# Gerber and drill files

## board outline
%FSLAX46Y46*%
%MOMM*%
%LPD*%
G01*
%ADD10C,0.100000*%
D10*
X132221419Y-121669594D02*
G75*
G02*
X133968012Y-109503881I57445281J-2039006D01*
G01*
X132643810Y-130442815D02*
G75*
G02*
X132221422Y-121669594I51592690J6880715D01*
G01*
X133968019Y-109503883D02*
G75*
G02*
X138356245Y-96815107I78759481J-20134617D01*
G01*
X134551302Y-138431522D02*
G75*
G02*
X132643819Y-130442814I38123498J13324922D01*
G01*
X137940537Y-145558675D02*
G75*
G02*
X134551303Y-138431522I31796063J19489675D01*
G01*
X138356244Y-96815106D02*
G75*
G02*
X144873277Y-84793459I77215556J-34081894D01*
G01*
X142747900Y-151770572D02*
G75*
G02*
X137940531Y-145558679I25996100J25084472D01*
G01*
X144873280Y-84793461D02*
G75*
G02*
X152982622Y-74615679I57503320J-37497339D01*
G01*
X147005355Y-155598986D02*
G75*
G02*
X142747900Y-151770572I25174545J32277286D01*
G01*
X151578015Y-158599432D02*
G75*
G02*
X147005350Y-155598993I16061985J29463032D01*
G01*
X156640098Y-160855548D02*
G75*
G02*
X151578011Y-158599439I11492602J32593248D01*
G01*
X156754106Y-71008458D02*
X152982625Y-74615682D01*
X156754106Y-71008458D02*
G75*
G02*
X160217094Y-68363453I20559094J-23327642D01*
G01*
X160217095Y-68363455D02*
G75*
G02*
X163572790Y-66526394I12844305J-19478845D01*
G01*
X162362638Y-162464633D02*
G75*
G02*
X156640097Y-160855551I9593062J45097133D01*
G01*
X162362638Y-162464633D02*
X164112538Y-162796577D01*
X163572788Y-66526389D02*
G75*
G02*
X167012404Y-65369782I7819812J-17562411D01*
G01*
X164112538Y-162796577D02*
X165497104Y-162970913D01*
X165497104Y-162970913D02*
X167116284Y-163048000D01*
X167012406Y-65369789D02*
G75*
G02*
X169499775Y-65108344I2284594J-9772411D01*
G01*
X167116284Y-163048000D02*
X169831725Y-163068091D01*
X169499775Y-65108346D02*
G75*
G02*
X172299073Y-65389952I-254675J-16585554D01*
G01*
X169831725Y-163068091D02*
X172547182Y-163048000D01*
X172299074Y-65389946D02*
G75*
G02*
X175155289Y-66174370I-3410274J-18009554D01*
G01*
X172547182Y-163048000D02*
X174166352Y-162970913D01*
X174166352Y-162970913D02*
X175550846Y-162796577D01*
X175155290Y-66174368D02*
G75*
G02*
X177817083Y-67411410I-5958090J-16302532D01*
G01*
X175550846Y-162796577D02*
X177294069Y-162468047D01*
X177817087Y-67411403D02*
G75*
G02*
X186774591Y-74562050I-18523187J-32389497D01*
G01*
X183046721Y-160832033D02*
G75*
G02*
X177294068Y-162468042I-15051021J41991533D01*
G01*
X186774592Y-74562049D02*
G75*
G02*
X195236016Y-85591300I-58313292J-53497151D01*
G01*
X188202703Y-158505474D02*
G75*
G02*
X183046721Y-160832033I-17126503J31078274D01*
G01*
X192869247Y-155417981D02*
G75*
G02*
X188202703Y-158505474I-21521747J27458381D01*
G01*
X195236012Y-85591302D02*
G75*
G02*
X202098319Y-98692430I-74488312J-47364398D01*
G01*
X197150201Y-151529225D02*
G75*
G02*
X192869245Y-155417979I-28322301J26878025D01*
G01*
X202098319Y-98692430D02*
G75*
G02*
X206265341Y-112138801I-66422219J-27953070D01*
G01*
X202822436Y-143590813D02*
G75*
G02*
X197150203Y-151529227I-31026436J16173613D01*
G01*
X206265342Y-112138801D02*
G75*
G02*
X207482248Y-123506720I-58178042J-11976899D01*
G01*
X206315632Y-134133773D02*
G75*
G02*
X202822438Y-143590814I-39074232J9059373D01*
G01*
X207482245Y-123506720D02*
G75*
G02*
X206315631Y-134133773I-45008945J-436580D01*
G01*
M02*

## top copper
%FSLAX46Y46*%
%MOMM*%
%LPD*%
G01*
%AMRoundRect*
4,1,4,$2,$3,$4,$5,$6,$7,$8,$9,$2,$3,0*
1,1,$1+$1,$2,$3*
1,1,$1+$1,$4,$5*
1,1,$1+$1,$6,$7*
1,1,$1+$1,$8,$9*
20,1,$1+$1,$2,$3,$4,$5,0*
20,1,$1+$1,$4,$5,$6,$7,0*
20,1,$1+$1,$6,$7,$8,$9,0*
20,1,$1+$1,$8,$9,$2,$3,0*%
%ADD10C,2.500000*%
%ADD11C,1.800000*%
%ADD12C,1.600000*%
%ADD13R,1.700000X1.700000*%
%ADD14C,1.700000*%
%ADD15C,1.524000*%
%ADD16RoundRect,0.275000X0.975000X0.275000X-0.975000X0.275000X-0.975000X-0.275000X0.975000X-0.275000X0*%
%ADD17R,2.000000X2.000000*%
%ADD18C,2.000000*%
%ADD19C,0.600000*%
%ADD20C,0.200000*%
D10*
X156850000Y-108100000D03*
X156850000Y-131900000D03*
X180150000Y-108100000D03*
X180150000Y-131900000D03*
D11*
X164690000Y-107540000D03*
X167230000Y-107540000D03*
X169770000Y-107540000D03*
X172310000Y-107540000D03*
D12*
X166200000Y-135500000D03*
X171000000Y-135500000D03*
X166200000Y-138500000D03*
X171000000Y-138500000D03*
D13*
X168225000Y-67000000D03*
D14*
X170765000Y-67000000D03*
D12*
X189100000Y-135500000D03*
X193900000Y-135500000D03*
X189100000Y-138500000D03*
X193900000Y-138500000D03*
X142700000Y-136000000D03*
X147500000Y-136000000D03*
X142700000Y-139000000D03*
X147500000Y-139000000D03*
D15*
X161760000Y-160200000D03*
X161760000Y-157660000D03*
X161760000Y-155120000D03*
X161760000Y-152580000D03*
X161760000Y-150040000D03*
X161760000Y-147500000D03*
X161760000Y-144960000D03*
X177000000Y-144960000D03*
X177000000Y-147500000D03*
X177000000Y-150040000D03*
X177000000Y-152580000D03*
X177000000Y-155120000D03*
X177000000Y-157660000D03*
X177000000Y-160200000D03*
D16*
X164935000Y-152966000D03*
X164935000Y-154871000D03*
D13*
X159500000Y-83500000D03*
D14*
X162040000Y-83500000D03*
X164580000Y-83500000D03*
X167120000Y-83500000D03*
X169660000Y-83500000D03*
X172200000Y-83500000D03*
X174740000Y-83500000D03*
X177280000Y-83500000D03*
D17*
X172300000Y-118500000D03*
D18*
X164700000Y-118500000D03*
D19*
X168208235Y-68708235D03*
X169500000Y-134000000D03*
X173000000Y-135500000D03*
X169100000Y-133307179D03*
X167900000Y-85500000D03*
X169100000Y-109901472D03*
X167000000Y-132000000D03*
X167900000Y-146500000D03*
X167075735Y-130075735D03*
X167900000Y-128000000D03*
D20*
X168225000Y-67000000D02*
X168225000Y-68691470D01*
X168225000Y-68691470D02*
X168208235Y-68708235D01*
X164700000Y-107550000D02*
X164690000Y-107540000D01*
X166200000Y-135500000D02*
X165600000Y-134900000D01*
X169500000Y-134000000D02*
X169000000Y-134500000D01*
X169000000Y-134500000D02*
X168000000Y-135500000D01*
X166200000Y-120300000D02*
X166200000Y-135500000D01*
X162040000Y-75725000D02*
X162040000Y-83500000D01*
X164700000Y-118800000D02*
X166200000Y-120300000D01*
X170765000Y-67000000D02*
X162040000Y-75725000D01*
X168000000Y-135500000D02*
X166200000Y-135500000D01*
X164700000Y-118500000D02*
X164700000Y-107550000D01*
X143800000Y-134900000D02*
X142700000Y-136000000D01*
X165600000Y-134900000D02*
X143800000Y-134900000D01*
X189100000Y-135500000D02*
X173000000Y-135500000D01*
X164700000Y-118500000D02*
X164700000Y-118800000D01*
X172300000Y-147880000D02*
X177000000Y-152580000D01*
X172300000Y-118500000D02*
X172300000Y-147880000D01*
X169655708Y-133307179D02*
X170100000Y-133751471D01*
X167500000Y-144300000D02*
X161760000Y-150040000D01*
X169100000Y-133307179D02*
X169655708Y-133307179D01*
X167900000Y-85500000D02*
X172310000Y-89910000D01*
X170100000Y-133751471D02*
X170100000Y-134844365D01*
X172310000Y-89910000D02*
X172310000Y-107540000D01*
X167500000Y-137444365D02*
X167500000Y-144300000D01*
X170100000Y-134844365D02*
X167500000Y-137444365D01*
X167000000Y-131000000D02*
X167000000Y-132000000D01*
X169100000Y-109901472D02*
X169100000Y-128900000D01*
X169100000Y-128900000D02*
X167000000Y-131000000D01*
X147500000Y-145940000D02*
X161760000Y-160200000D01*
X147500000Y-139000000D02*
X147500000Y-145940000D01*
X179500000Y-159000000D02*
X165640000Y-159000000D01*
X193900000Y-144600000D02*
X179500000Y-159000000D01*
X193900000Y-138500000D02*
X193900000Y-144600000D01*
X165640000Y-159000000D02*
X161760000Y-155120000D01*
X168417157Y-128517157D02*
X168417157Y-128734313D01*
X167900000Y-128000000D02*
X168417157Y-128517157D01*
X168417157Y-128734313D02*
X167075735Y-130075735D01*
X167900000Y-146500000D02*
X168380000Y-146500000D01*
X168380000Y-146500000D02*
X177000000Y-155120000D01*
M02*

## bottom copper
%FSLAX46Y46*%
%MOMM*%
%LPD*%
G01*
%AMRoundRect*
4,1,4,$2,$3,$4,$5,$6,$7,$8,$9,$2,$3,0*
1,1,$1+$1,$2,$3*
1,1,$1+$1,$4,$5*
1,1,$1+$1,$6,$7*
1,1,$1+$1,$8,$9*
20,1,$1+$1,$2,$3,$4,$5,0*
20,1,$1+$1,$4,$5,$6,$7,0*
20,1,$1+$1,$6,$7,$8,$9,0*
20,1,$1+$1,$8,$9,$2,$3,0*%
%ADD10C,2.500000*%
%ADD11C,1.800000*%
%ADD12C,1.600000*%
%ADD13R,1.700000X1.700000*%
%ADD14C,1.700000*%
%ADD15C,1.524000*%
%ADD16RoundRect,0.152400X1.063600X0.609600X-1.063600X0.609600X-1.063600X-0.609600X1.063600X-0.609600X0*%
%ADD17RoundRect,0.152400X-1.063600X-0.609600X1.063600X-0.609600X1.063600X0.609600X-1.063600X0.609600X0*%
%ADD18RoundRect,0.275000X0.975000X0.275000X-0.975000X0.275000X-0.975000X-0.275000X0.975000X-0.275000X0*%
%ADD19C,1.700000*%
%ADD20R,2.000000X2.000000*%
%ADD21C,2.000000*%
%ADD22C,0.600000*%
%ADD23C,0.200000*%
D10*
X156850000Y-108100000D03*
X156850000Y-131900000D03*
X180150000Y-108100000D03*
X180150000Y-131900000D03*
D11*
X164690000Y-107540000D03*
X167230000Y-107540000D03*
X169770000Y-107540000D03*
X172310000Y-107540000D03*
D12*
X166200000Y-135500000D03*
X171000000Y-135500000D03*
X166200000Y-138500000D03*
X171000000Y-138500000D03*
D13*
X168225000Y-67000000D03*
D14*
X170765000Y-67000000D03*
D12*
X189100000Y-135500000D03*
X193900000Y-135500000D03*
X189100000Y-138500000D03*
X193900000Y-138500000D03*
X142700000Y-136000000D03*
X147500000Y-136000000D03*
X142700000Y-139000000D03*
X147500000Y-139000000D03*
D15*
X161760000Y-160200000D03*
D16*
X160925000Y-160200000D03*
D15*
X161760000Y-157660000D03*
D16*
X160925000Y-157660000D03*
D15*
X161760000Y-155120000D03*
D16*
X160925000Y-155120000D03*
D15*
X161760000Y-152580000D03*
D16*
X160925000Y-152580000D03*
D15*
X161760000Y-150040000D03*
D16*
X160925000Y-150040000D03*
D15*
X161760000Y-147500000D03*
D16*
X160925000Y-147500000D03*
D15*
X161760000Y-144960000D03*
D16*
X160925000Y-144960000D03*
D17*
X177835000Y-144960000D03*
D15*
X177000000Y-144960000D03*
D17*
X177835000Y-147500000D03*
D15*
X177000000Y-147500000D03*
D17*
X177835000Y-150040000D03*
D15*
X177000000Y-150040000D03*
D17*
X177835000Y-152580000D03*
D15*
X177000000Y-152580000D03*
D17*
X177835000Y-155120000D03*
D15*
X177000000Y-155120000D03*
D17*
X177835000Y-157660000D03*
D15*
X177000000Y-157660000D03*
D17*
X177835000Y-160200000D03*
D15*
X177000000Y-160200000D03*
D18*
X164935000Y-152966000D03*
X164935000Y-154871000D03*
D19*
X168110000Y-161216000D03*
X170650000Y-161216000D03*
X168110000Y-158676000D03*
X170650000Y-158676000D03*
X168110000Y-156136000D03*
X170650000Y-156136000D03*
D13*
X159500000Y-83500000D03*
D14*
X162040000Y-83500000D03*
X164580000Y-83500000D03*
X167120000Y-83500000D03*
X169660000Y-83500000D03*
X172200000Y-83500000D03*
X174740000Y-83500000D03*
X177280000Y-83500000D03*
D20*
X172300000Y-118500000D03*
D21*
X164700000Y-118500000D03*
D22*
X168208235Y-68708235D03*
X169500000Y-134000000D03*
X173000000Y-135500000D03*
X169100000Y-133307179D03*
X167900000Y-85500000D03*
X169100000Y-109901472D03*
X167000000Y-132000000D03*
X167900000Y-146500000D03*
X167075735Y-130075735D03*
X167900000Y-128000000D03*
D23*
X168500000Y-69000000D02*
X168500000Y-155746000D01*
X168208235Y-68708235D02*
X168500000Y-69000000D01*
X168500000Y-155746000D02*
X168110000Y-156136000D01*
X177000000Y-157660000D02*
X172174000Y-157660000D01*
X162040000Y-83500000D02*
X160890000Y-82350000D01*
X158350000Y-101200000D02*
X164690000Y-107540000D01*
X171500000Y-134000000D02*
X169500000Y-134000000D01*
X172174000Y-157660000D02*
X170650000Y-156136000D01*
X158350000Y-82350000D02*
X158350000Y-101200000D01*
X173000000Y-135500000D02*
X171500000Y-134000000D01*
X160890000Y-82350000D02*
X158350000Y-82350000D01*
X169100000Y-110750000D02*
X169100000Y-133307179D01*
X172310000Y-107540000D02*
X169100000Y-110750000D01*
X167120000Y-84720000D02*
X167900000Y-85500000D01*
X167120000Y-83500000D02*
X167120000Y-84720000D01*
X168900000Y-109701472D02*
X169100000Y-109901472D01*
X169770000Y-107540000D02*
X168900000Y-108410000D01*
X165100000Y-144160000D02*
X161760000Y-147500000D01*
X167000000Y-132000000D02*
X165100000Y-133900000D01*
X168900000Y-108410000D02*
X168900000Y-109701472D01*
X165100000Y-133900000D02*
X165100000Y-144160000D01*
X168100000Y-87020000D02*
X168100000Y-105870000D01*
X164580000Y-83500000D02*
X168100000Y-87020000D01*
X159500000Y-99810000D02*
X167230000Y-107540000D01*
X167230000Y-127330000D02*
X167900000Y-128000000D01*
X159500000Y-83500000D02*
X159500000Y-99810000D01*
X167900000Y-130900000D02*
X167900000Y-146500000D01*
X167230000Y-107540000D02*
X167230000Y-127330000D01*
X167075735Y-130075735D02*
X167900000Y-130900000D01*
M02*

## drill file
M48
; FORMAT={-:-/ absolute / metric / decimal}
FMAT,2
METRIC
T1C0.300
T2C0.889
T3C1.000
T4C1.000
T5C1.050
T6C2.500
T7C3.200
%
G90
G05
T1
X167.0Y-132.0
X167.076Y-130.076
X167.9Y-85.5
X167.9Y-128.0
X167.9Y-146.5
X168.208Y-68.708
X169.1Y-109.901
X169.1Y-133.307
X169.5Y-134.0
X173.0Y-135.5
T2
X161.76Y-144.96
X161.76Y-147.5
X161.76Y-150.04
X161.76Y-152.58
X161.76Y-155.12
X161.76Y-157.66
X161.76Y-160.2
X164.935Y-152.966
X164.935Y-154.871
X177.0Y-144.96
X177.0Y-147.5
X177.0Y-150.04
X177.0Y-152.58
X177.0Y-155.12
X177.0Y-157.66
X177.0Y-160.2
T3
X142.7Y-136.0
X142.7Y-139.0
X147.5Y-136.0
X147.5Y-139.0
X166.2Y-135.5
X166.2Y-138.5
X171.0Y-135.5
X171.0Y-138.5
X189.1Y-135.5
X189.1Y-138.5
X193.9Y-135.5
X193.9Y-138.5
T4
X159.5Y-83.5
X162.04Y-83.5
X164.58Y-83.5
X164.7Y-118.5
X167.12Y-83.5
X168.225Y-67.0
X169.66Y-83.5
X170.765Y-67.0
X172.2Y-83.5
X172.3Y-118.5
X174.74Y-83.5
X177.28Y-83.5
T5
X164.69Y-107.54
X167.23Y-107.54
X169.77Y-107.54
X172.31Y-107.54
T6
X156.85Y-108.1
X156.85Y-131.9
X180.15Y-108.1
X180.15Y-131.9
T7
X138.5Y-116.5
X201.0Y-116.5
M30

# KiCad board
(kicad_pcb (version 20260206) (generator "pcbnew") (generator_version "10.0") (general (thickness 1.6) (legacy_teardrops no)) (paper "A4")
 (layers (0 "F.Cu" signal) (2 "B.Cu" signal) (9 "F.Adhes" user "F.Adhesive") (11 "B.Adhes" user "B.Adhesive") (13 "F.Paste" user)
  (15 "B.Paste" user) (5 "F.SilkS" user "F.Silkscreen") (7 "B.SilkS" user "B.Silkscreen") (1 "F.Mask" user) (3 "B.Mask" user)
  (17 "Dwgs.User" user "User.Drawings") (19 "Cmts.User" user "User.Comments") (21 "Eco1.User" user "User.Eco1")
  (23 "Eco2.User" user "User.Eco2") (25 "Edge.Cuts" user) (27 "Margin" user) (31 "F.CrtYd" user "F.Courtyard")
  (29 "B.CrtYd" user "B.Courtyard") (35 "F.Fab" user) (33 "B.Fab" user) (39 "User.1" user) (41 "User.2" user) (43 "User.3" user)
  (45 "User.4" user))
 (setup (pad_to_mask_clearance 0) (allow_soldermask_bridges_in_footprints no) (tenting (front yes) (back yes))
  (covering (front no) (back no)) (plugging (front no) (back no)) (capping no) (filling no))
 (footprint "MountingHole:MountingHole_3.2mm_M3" (layer "F.Cu") (at 138.5 116.5)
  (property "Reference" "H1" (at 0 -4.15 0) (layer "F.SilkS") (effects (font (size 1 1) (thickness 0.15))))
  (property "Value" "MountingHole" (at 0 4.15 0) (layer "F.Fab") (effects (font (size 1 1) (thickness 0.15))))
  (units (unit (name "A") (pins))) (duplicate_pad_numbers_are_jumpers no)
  (pad "" np_thru_hole circle (at 0 0) (size 3.2 3.2) (drill 3.2) (layers "*.Cu" "*.Mask")))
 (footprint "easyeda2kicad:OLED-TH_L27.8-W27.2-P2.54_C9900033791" (layer "F.Cu") (at 168.5 107.54)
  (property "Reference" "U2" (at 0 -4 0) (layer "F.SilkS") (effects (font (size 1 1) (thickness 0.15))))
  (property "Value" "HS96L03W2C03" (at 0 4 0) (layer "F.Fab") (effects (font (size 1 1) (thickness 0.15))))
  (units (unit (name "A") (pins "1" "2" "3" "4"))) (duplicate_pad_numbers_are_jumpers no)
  (pad "" thru_hole circle (at -11.65 0.56) (size 2.5 2.5) (drill 2.5) (layers "*.Cu" "*.Mask") (remove_unused_layers no))
  (pad "" thru_hole circle (at -11.65 24.36) (size 2.5 2.5) (drill 2.5) (layers "*.Cu" "*.Mask") (remove_unused_layers no))
  (pad "" thru_hole circle (at 11.65 0.56) (size 2.5 2.5) (drill 2.5) (layers "*.Cu" "*.Mask") (remove_unused_layers no))
  (pad "" thru_hole circle (at 11.65 24.36) (size 2.5 2.5) (drill 2.5) (layers "*.Cu" "*.Mask") (remove_unused_layers no))
  (pad "1" thru_hole circle (at -3.81 0) (size 1.8 1.8) (drill 1.049986) (layers "*.Cu" "*.Mask") (remove_unused_layers no) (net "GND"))
  (pad "2" thru_hole circle (at -1.27 0) (size 1.8 1.8) (drill 1.049986) (layers "*.Cu" "*.Mask") (remove_unused_layers no) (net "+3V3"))
  (pad "3" thru_hole circle (at 1.27 0) (size 1.8 1.8) (drill 1.049986) (layers "*.Cu" "*.Mask") (remove_unused_layers no) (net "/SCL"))
  (pad "4" thru_hole circle (at 3.81 0) (size 1.8 1.8) (drill 1.049986) (layers "*.Cu" "*.Mask") (remove_unused_layers no) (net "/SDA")))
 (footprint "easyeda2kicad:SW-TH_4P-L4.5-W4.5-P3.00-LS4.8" (layer "F.Cu") (at 168.6 137)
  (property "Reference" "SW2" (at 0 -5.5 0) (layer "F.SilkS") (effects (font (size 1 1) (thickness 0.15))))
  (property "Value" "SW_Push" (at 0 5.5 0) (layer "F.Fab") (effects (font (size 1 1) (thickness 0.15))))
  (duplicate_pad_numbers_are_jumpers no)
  (pad "1" thru_hole circle (at -2.4 -1.5) (size 1.6 1.6) (drill 0.999998) (layers "*.Cu" "*.Mask") (remove_unused_layers no) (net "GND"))
  (pad "1" thru_hole circle (at 2.4 -1.5) (size 1.6 1.6) (drill 0.999998) (layers "*.Cu" "*.Mask") (remove_unused_layers no))
  (pad "2" thru_hole circle (at -2.4 1.5) (size 1.6 1.6) (drill 0.999998) (layers "*.Cu" "*.Mask") (remove_unused_layers no))
  (pad "2" thru_hole circle (at 2.4 1.5) (size 1.6 1.6) (drill 0.999998) (layers "*.Cu" "*.Mask") (remove_unused_layers no)
   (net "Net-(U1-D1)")))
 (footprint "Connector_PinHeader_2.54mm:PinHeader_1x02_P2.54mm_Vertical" (layer "F.Cu") (at 168.225 67 90)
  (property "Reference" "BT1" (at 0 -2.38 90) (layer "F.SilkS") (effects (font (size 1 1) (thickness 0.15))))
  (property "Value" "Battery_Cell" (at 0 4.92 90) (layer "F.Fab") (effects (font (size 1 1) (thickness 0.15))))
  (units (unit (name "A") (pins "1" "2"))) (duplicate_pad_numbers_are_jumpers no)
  (pad "1" thru_hole rect (at 0 0 90) (size 1.7 1.7) (drill 1) (layers "*.Cu" "*.Mask") (remove_unused_layers no) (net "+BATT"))
  (pad "2" thru_hole circle (at 0 2.54 90) (size 1.7 1.7) (drill 1) (layers "*.Cu" "*.Mask") (remove_unused_layers no) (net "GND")))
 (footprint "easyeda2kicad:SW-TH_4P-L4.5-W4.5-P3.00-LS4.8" (layer "F.Cu") (at 191.5 137)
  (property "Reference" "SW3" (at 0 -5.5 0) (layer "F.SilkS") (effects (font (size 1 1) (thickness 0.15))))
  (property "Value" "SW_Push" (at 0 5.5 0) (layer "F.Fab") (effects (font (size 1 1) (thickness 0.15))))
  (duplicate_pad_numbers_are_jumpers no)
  (pad "1" thru_hole circle (at -2.4 -1.5) (size 1.6 1.6) (drill 0.999998) (layers "*.Cu" "*.Mask") (remove_unused_layers no) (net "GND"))
  (pad "1" thru_hole circle (at 2.4 -1.5) (size 1.6 1.6) (drill 0.999998) (layers "*.Cu" "*.Mask") (remove_unused_layers no))
  (pad "2" thru_hole circle (at -2.4 1.5) (size 1.6 1.6) (drill 0.999998) (layers "*.Cu" "*.Mask") (remove_unused_layers no))
  (pad "2" thru_hole circle (at 2.4 1.5) (size 1.6 1.6) (drill 0.999998) (layers "*.Cu" "*.Mask") (remove_unused_layers no)
   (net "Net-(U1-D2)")))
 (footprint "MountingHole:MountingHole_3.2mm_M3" (layer "F.Cu") (at 201 116.5)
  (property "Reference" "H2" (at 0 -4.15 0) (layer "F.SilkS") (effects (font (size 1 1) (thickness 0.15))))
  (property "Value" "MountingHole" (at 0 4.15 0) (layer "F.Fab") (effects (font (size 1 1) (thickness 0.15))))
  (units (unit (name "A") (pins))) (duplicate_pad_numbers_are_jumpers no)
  (pad "" np_thru_hole circle (at 0 0) (size 3.2 3.2) (drill 3.2) (layers "*.Cu" "*.Mask")))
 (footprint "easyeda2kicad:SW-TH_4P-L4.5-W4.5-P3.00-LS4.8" (layer "F.Cu") (at 145.1 137.5)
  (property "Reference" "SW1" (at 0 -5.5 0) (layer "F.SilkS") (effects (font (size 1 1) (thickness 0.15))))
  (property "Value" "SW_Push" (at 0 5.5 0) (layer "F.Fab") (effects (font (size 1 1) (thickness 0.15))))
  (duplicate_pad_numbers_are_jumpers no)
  (pad "1" thru_hole circle (at -2.4 -1.5) (size 1.6 1.6) (drill 0.999998) (layers "*.Cu" "*.Mask") (remove_unused_layers no) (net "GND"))
  (pad "1" thru_hole circle (at 2.4 -1.5) (size 1.6 1.6) (drill 0.999998) (layers "*.Cu" "*.Mask") (remove_unused_layers no))
  (pad "2" thru_hole circle (at -2.4 1.5) (size 1.6 1.6) (drill 0.999998) (layers "*.Cu" "*.Mask") (remove_unused_layers no))
  (pad "2" thru_hole circle (at 2.4 1.5) (size 1.6 1.6) (drill 0.999998) (layers "*.Cu" "*.Mask") (remove_unused_layers no)
   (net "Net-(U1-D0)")))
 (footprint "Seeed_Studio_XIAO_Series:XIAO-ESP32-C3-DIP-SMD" (layer "B.Cu") (at 169.38 152.58 -90)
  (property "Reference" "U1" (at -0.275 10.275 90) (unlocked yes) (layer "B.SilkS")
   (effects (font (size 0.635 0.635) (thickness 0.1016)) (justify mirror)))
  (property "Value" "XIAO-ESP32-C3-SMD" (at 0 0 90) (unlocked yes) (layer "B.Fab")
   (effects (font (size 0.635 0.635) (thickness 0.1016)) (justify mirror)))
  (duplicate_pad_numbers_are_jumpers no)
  (pad "1" thru_hole circle (at 7.62 7.62 180) (size 1.524 1.524) (drill 0.889) (layers "*.Cu" "*.Mask") (remove_unused_layers no)
   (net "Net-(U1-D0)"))
  (pad "1" smd roundrect (at 7.62 8.455 180) (size 2.432 1.524) (layers "B.Cu" "B.Mask") (roundrect_rratio 0.1) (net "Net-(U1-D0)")
   (thermal_bridge_angle 45))
  (pad "2" thru_hole circle (at 5.08 7.62 180) (size 1.524 1.524) (drill 0.889) (layers "*.Cu" "*.Mask") (remove_unused_layers no)
   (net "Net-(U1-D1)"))
  (pad "2" smd roundrect (at 5.08 8.455 180) (size 2.432 1.524) (layers "B.Cu" "B.Mask") (roundrect_rratio 0.1) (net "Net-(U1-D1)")
   (thermal_bridge_angle 45))
  (pad "3" thru_hole circle (at 2.54 7.62 180) (size 1.524 1.524) (drill 0.889) (layers "*.Cu" "*.Mask") (remove_unused_layers no)
   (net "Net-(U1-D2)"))
  (pad "3" smd roundrect (at 2.54 8.455 180) (size 2.432 1.524) (layers "B.Cu" "B.Mask") (roundrect_rratio 0.1) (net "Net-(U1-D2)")
   (thermal_bridge_angle 45))
  (pad "4" thru_hole circle (at 0 7.62 180) (size 1.524 1.524) (drill 0.889) (layers "*.Cu" "*.Mask") (remove_unused_layers no)
   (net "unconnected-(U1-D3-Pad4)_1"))
  (pad "4" smd roundrect (at 0 8.455 180) (size 2.432 1.524) (layers "B.Cu" "B.Mask") (roundrect_rratio 0.1)
   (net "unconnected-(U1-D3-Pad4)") (thermal_bridge_angle 45))
  (pad "5" thru_hole circle (at -2.54 7.62 180) (size 1.524 1.524) (drill 0.889) (layers "*.Cu" "*.Mask") (remove_unused_layers no)
   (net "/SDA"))
  (pad "5" smd roundrect (at -2.54 8.455 180) (size 2.432 1.524) (layers "B.Cu" "B.Mask") (roundrect_rratio 0.1) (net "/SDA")
   (thermal_bridge_angle 45))
  (pad "6" thru_hole circle (at -5.08 7.62 180) (size 1.524 1.524) (drill 0.889) (layers "*.Cu" "*.Mask") (remove_unused_layers no)
   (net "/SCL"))
  (pad "6" smd roundrect (at -5.08 8.455 180) (size 2.432 1.524) (layers "B.Cu" "B.Mask") (roundrect_rratio 0.1) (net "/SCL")
   (thermal_bridge_angle 45))
  (pad "7" thru_hole circle (at -7.62 7.62 180) (size 1.524 1.524) (drill 0.889) (layers "*.Cu" "*.Mask") (remove_unused_layers no)
   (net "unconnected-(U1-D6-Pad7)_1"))
  (pad "7" smd roundrect (at -7.62 8.455 180) (size 2.432 1.524) (layers "B.Cu" "B.Mask") (roundrect_rratio 0.1)
   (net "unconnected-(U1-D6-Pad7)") (thermal_bridge_angle 45))
  (pad "8" smd roundrect (at -7.62 -8.455) (size 2.432 1.524) (layers "B.Cu" "B.Mask") (roundrect_rratio 0.1)
   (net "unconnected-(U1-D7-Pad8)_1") (thermal_bridge_angle 45))
  (pad "8" thru_hole circle (at -7.62 -7.62) (size 1.524 1.524) (drill 0.889) (layers "*.Cu" "*.Mask") (remove_unused_layers no)
   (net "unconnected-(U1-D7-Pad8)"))
  (pad "9" smd roundrect (at -5.08 -8.455) (size 2.432 1.524) (layers "B.Cu" "B.Mask") (roundrect_rratio 0.1)
   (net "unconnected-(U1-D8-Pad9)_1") (thermal_bridge_angle 45))
  (pad "9" thru_hole circle (at -5.08 -7.62) (size 1.524 1.524) (drill 0.889) (layers "*.Cu" "*.Mask") (remove_unused_layers no)
   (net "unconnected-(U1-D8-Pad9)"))
  (pad "10" smd roundrect (at -2.54 -8.455) (size 2.432 1.524) (layers "B.Cu" "B.Mask") (roundrect_rratio 0.1)
   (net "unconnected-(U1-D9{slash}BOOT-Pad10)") (thermal_bridge_angle 45))
  (pad "10" thru_hole circle (at -2.54 -7.62) (size 1.524 1.524) (drill 0.889) (layers "*.Cu" "*.Mask") (remove_unused_layers no)
   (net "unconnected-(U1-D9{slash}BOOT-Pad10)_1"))
  (pad "11" smd roundrect (at 0 -8.455) (size 2.432 1.524) (layers "B.Cu" "B.Mask") (roundrect_rratio 0.1) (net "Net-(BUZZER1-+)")
   (thermal_bridge_angle 45))
  (pad "11" thru_hole circle (at 0 -7.62) (size 1.524 1.524) (drill 0.889) (layers "*.Cu" "*.Mask") (remove_unused_layers no)
   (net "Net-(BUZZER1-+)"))
  (pad "12" smd roundrect (at 2.54 -8.455) (size 2.432 1.524) (layers "B.Cu" "B.Mask") (roundrect_rratio 0.1) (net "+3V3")
   (thermal_bridge_angle 45))
  (pad "12" thru_hole circle (at 2.54 -7.62) (size 1.524 1.524) (drill 0.889) (layers "*.Cu" "*.Mask") (remove_unused_layers no)
   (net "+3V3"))
  (pad "13" smd roundrect (at 5.08 -8.455) (size 2.432 1.524) (layers "B.Cu" "B.Mask") (roundrect_rratio 0.1) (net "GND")
   (thermal_bridge_angle 45))
  (pad "13" thru_hole circle (at 5.08 -7.62) (size 1.524 1.524) (drill 0.889) (layers "*.Cu" "*.Mask") (remove_unused_layers no) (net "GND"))
  (pad "14" smd roundrect (at 7.62 -8.455) (size 2.432 1.524) (layers "B.Cu" "B.Mask") (roundrect_rratio 0.1) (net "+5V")
   (thermal_bridge_angle 45))
  (pad "14" thru_hole circle (at 7.62 -7.62) (size 1.524 1.524) (drill 0.889) (layers "*.Cu" "*.Mask") (remove_unused_layers no) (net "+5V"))
  (pad "15" thru_hole roundrect (at 0.386 4.445 180) (size 2.5 1.1) (drill 0.889) (layers "*.Cu" "B.Mask" "B.Paste")
   (remove_unused_layers no) (roundrect_rratio 0.25) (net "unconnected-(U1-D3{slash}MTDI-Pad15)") (thermal_bridge_angle 45))
  (pad "16" thru_hole roundrect (at 2.291 4.445 180) (size 2.5 1.1) (drill 0.889) (layers "*.Cu" "*.Mask") (remove_unused_layers no)
   (roundrect_rratio 0.25) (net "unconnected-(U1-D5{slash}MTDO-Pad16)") (thermal_bridge_angle 45))
  (pad "17" smd circle (at 8.636 1.27) (size 1.7 1.7) (layers "B.Cu" "B.Mask" "B.Paste") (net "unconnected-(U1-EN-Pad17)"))
  (pad "18" smd circle (at 8.636 -1.27) (size 1.7 1.7) (layers "B.Cu" "B.Mask" "B.Paste") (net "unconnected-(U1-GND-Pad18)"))
  (pad "19" smd circle (at 6.096 1.27) (size 1.7 1.7) (layers "B.Cu" "B.Mask" "B.Paste") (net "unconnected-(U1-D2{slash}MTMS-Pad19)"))
  (pad "20" smd circle (at 6.096 -1.27) (size 1.7 1.7) (layers "B.Cu" "B.Mask" "B.Paste") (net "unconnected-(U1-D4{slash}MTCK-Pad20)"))
  (pad "21" smd circle (at 3.556 1.27) (size 1.7 1.7) (layers "B.Cu" "B.Mask" "B.Paste") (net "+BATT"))
  (pad "22" smd circle (at 3.556 -1.27) (size 1.7 1.7) (layers "B.Cu" "B.Mask" "B.Paste") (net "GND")))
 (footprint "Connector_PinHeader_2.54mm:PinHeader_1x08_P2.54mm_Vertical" (layer "B.Cu") (at 159.5 83.5 -90)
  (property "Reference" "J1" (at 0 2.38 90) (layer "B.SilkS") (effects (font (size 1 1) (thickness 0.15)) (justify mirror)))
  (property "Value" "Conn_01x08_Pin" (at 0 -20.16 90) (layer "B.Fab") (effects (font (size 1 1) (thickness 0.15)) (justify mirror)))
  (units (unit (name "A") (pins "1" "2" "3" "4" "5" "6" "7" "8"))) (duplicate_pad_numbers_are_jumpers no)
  (pad "1" thru_hole rect (at 0 0 270) (size 1.7 1.7) (drill 1) (layers "*.Cu" "*.Mask") (remove_unused_layers no) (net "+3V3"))
  (pad "2" thru_hole circle (at 0 -2.54 270) (size 1.7 1.7) (drill 1) (layers "*.Cu" "*.Mask") (remove_unused_layers no) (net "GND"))
  (pad "3" thru_hole circle (at 0 -5.08 270) (size 1.7 1.7) (drill 1) (layers "*.Cu" "*.Mask") (remove_unused_layers no) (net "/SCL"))
  (pad "4" thru_hole circle (at 0 -7.62 270) (size 1.7 1.7) (drill 1) (layers "*.Cu" "*.Mask") (remove_unused_layers no) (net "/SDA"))
  (pad "5" thru_hole circle (at 0 -10.16 270) (size 1.7 1.7) (drill 1) (layers "*.Cu" "*.Mask") (remove_unused_layers no)
   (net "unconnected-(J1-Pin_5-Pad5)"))
  (pad "6" thru_hole circle (at 0 -12.7 270) (size 1.7 1.7) (drill 1) (layers "*.Cu" "*.Mask") (remove_unused_layers no)
   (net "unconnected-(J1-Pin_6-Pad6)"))
  (pad "7" thru_hole circle (at 0 -15.24 270) (size 1.7 1.7) (drill 1) (layers "*.Cu" "*.Mask") (remove_unused_layers no)
   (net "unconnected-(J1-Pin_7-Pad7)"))
  (pad "8" thru_hole circle (at 0 -17.78 270) (size 1.7 1.7) (drill 1) (layers "*.Cu" "*.Mask") (remove_unused_layers no)
   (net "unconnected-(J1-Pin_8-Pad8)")))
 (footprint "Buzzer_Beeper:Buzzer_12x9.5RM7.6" (layer "B.Cu") (at 172.3 118.5 180)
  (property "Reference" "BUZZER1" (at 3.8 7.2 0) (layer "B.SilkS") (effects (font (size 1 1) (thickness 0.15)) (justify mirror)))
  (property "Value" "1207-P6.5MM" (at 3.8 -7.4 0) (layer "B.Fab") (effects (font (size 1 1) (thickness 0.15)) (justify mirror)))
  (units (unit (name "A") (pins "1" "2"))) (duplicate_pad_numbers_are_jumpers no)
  (pad "1" thru_hole rect (at 0 0 180) (size 2 2) (drill 1) (layers "*.Cu" "*.Mask") (remove_unused_layers no) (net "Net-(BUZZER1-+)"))
  (pad "2" thru_hole circle (at 7.6 0 180) (size 2 2) (drill 1) (layers "*.Cu" "*.Mask") (remove_unused_layers no) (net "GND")))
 (gr_arc (start 132.221419 121.669594) (mid 132.768623 115.539984) (end 133.968019 109.503883) (stroke (width 0) (type default))
  (layer "Edge.Cuts"))
 (gr_arc (start 132.64381 130.442815) (mid 132.24722 126.065067) (end 132.221419 121.669594) (stroke (width 0) (type default))
  (layer "Edge.Cuts"))
 (gr_arc (start 133.968019 109.503883) (mid 135.899728 103.068738) (end 138.356244 96.815106) (stroke (width 0) (type default))
  (layer "Edge.Cuts"))
 (gr_arc (start 134.551302 138.431522) (mid 133.393946 134.485807) (end 132.64381 130.442815) (stroke (width 0) (type default))
  (layer "Edge.Cuts"))
 (gr_arc (start 137.940537 145.558675) (mid 136.056908 142.085099) (end 134.551302 138.431522) (stroke (width 0) (type default))
  (layer "Edge.Cuts"))
 (gr_arc (start 138.356244 96.815106) (mid 141.370886 90.672111) (end 144.87328 84.793461) (stroke (width 0) (type default))
  (layer "Edge.Cuts"))
 (gr_arc (start 142.7479 151.770572) (mid 140.17485 148.795631) (end 137.940537 145.558675) (stroke (width 0) (type default))
  (layer "Edge.Cuts"))
 (gr_arc (start 144.87328 84.793461) (mid 148.686299 79.511909) (end 152.982625 74.615682) (stroke (width 0) (type default))
  (layer "Edge.Cuts"))
 (gr_arc (start 147.005355 155.598986) (mid 144.809638 153.759336) (end 142.7479 151.770572) (stroke (width 0) (type default))
  (layer "Edge.Cuts"))
 (gr_arc (start 151.578015 158.599432) (mid 149.230446 157.192516) (end 147.005355 155.598986) (stroke (width 0) (type default))
  (layer "Edge.Cuts"))
 (gr_arc (start 156.640098 160.855548) (mid 154.063749 159.829119) (end 151.578015 158.599432) (stroke (width 0) (type default))
  (layer "Edge.Cuts"))
 (gr_line (start 156.754106 71.008458) (end 152.982625 74.615682) (stroke (width 0) (type default)) (layer "Edge.Cuts"))
 (gr_arc (start 156.754106 71.008458) (mid 158.43922 69.625211) (end 160.217095 68.363455) (stroke (width 0) (type default))
  (layer "Edge.Cuts"))
 (gr_arc (start 160.217095 68.363455) (mid 161.857242 67.376022) (end 163.572788 66.526389) (stroke (width 0) (type default))
  (layer "Edge.Cuts"))
 (gr_arc (start 162.362638 162.464633) (mid 159.475425 161.752417) (end 156.640098 160.855548) (stroke (width 0) (type default))
  (layer "Edge.Cuts"))
 (gr_line (start 162.362638 162.464633) (end 164.112538 162.796577) (stroke (width 0) (type default)) (layer "Edge.Cuts"))
 (gr_arc (start 163.572788 66.526389) (mid 165.265193 65.866767) (end 167.012406 65.369789) (stroke (width 0) (type default))
  (layer "Edge.Cuts"))
 (gr_line (start 164.112538 162.796577) (end 165.497104 162.970913) (stroke (width 0) (type default)) (layer "Edge.Cuts"))
 (gr_line (start 165.497104 162.970913) (end 167.116284 163.048) (stroke (width 0) (type default)) (layer "Edge.Cuts"))
 (gr_arc (start 167.012406 65.369789) (mid 168.248044 65.161265) (end 169.499775 65.108346) (stroke (width 0) (type default))
  (layer "Edge.Cuts"))
 (gr_line (start 167.116284 163.048) (end 169.831725 163.068091) (stroke (width 0) (type default)) (layer "Edge.Cuts"))
 (gr_arc (start 169.499775 65.108346) (mid 170.905379 65.189687) (end 172.299074 65.389946) (stroke (width 0) (type default))
  (layer "Edge.Cuts"))
 (gr_line (start 169.831725 163.068091) (end 172.547182 163.048) (stroke (width 0) (type default)) (layer "Edge.Cuts"))
 (gr_arc (start 172.299074 65.389946) (mid 173.743021 65.72436) (end 175.15529 66.174368) (stroke (width 0) (type default))
  (layer "Edge.Cuts"))
 (gr_line (start 172.547182 163.048) (end 174.166352 162.970913) (stroke (width 0) (type default)) (layer "Edge.Cuts"))
 (gr_line (start 174.166352 162.970913) (end 175.550846 162.796577) (stroke (width 0) (type default)) (layer "Edge.Cuts"))
 (gr_arc (start 175.15529 66.174368) (mid 176.512389 66.736521) (end 177.817087 67.411403) (stroke (width 0) (type default))
  (layer "Edge.Cuts"))
 (gr_line (start 175.550846 162.796577) (end 177.294069 162.468047) (stroke (width 0) (type default)) (layer "Edge.Cuts"))
 (gr_arc (start 177.817087 67.411403) (mid 182.571982 70.640671) (end 186.774592 74.562049) (stroke (width 0) (type default))
  (layer "Edge.Cuts"))
 (gr_arc (start 183.046721 160.832033) (mid 180.197865 161.746554) (end 177.294069 162.468047) (stroke (width 0) (type default))
  (layer "Edge.Cuts"))
 (gr_arc (start 186.774592 74.562049) (mid 191.247953 79.890527) (end 195.236012 85.591302) (stroke (width 0) (type default))
  (layer "Edge.Cuts"))
 (gr_arc (start 188.202703 158.505474) (mid 185.671133 159.771661) (end 183.046721 160.832033) (stroke (width 0) (type default))
  (layer "Edge.Cuts"))
 (gr_arc (start 192.869247 155.417981) (mid 190.597996 157.055419) (end 188.202703 158.505474) (stroke (width 0) (type default))
  (layer "Edge.Cuts"))
 (gr_arc (start 195.236012 85.591302) (mid 198.942007 91.997853) (end 202.098319 98.69243) (stroke (width 0) (type default))
  (layer "Edge.Cuts"))
 (gr_arc (start 197.150201 151.529225) (mid 195.08178 153.553014) (end 192.869247 155.417981) (stroke (width 0) (type default))
  (layer "Edge.Cuts"))
 (gr_arc (start 202.098319 98.69243) (mid 204.510968 105.313686) (end 206.265342 112.138801) (stroke (width 0) (type default))
  (layer "Edge.Cuts"))
 (gr_arc (start 202.822436 143.590813) (mid 200.264346 147.75875) (end 197.150201 151.529225) (stroke (width 0) (type default))
  (layer "Edge.Cuts"))
 (gr_arc (start 206.265342 112.138801) (mid 207.147932 117.793337) (end 207.482245 123.50672) (stroke (width 0) (type default))
  (layer "Edge.Cuts"))
 (gr_arc (start 206.315632 134.133773) (mid 204.867371 138.972388) (end 202.822436 143.590813) (stroke (width 0) (type default))
  (layer "Edge.Cuts"))
 (gr_arc (start 207.482245 123.50672) (mid 207.215562 128.855096) (end 206.315632 134.133773) (stroke (width 0) (type default))
  (layer "Edge.Cuts"))
 (segment (start 168.225 67) (end 168.225 68.69147) (width 0.2) (layer "F.Cu") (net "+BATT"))
 (segment (start 168.225 68.69147) (end 168.208235 68.708235) (width 0.2) (layer "F.Cu") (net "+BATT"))
 (via (at 168.208235 68.708235) (size 0.6) (drill 0.3) (layers "F.Cu" "B.Cu") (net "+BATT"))
 (segment (start 168.5 69) (end 168.5 155.746) (width 0.2) (layer "B.Cu") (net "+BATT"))
 (segment (start 168.208235 68.708235) (end 168.5 69) (width 0.2) (layer "B.Cu") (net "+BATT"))
 (segment (start 168.5 155.746) (end 168.11 156.136) (width 0.2) (layer "B.Cu") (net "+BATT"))
 (segment (start 164.7 107.55) (end 164.69 107.54) (width 0.2) (layer "F.Cu") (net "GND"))
 (segment (start 166.2 135.5) (end 165.6 134.9) (width 0.2) (layer "F.Cu") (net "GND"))
 (segment (start 169.5 134) (end 169 134.5) (width 0.2) (layer "F.Cu") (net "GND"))
 (segment (start 169 134.5) (end 168 135.5) (width 0.2) (layer "F.Cu") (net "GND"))
 (segment (start 166.2 120.3) (end 166.2 135.5) (width 0.2) (layer "F.Cu") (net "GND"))
 (segment (start 162.04 75.725) (end 162.04 83.5) (width 0.2) (layer "F.Cu") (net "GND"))
 (segment (start 164.7 118.8) (end 166.2 120.3) (width 0.2) (layer "F.Cu") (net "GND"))
 (segment (start 170.765 67) (end 162.04 75.725) (width 0.2) (layer "F.Cu") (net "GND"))
 (segment (start 168 135.5) (end 166.2 135.5) (width 0.2) (layer "F.Cu") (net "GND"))
 (segment (start 164.7 118.5) (end 164.7 107.55) (width 0.2) (layer "F.Cu") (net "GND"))
 (segment (start 143.8 134.9) (end 142.7 136) (width 0.2) (layer "F.Cu") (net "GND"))
 (segment (start 165.6 134.9) (end 143.8 134.9) (width 0.2) (layer "F.Cu") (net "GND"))
 (segment (start 189.1 135.5) (end 173 135.5) (width 0.2) (layer "F.Cu") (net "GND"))
 (segment (start 164.7 118.5) (end 164.7 118.8) (width 0.2) (layer "F.Cu") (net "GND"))
 (via (at 169.5 134) (size 0.6) (drill 0.3) (layers "F.Cu" "B.Cu") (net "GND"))
 (via (at 173 135.5) (size 0.6) (drill 0.3) (layers "F.Cu" "B.Cu") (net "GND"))
 (segment (start 177 157.66) (end 172.174 157.66) (width 0.2) (layer "B.Cu") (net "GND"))
 (segment (start 162.04 83.5) (end 160.89 82.35) (width 0.2) (layer "B.Cu") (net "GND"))
 (segment (start 158.35 101.2) (end 164.69 107.54) (width 0.2) (layer "B.Cu") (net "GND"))
 (segment (start 171.5 134) (end 169.5 134) (width 0.2) (layer "B.Cu") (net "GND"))
 (segment (start 172.174 157.66) (end 170.65 156.136) (width 0.2) (layer "B.Cu") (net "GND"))
 (segment (start 158.35 82.35) (end 158.35 101.2) (width 0.2) (layer "B.Cu") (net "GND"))
 (segment (start 173 135.5) (end 171.5 134) (width 0.2) (layer "B.Cu") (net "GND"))
 (segment (start 160.89 82.35) (end 158.35 82.35) (width 0.2) (layer "B.Cu") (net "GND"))
 (segment (start 172.3 147.88) (end 177 152.58) (width 0.2) (layer "F.Cu") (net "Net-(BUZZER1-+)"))
 (segment (start 172.3 118.5) (end 172.3 147.88) (width 0.2) (layer "F.Cu") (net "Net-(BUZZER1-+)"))
 (segment (start 169.655708 133.307179) (end 170.1 133.751471) (width 0.2) (layer "F.Cu") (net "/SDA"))
 (segment (start 167.5 144.3) (end 161.76 150.04) (width 0.2) (layer "F.Cu") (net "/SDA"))
 (segment (start 169.1 133.307179) (end 169.655708 133.307179) (width 0.2) (layer "F.Cu") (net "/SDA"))
 (segment (start 167.9 85.5) (end 172.31 89.91) (width 0.2) (layer "F.Cu") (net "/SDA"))
 (segment (start 170.1 133.751471) (end 170.1 134.844365) (width 0.2) (layer "F.Cu") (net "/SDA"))
 (segment (start 172.31 89.91) (end 172.31 107.54) (width 0.2) (layer "F.Cu") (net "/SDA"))
 (segment (start 167.5 137.444365) (end 167.5 144.3) (width 0.2) (layer "F.Cu") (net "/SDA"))
 (segment (start 170.1 134.844365) (end 167.5 137.444365) (width 0.2) (layer "F.Cu") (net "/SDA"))
 (via (at 169.1 133.307179) (size 0.6) (drill 0.3) (layers "F.Cu" "B.Cu") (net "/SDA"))
 (via (at 167.9 85.5) (size 0.6) (drill 0.3) (layers "F.Cu" "B.Cu") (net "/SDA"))
 (segment (start 169.1 110.75) (end 169.1 133.307179) (width 0.2) (layer "B.Cu") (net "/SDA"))
 (segment (start 172.31 107.54) (end 169.1 110.75) (width 0.2) (layer "B.Cu") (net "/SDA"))
 (segment (start 167.12 84.72) (end 167.9 85.5) (width 0.2) (layer "B.Cu") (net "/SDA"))
 (segment (start 167.12 83.5) (end 167.12 84.72) (width 0.2) (layer "B.Cu") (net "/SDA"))
 (segment (start 167 131) (end 167 132) (width 0.2) (layer "F.Cu") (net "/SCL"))
 (segment (start 169.1 109.901472) (end 169.1 128.9) (width 0.2) (layer "F.Cu") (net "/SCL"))
 (segment (start 169.1 128.9) (end 167 131) (width 0.2) (layer "F.Cu") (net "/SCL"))
 (via (at 169.1 109.901472) (size 0.6) (drill 0.3) (layers "F.Cu" "B.Cu") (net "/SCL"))
 (via (at 167 132) (size 0.6) (drill 0.3) (layers "F.Cu" "B.Cu") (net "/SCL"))
 (segment (start 168.9 109.701472) (end 169.1 109.901472) (width 0.2) (layer "B.Cu") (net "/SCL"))
 (segment (start 169.77 107.54) (end 168.9 108.41) (width 0.2) (layer "B.Cu") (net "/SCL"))
 (segment (start 165.1 144.16) (end 161.76 147.5) (width 0.2) (layer "B.Cu") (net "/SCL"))
 (segment (start 167 132) (end 165.1 133.9) (width 0.2) (layer "B.Cu") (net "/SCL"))
 (segment (start 168.9 108.41) (end 168.9 109.701472) (width 0.2) (layer "B.Cu") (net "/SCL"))
 (segment (start 165.1 133.9) (end 165.1 144.16) (width 0.2) (layer "B.Cu") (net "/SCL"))
 (segment (start 168.1 87.02) (end 168.1 105.87) (width 0.2) (layer "B.Cu") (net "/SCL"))
 (segment (start 164.58 83.5) (end 168.1 87.02) (width 0.2) (layer "B.Cu") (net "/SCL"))
 (segment (start 147.5 145.94) (end 161.76 160.2) (width 0.2) (layer "F.Cu") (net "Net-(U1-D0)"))
 (segment (start 147.5 139) (end 147.5 145.94) (width 0.2) (layer "F.Cu") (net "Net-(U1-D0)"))
 (segment (start 179.5 159) (end 165.64 159) (width 0.2) (layer "F.Cu") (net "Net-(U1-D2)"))
 (segment (start 193.9 144.6) (end 179.5 159) (width 0.2) (layer "F.Cu") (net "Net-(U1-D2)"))
 (segment (start 193.9 138.5) (end 193.9 144.6) (width 0.2) (layer "F.Cu") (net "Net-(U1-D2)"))
 (segment (start 165.64 159) (end 161.76 155.12) (width 0.2) (layer "F.Cu") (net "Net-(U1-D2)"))
 (segment (start 168.417157 128.517157) (end 168.417157 128.734313) (width 0.2) (layer "F.Cu") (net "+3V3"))
 (segment (start 167.9 128) (end 168.417157 128.517157) (width 0.2) (layer "F.Cu") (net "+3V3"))
 (segment (start 168.417157 128.734313) (end 167.075735 130.075735) (width 0.2) (layer "F.Cu") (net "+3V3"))
 (segment (start 167.9 146.5) (end 168.38 146.5) (width 0.2) (layer "F.Cu") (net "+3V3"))
 (segment (start 168.38 146.5) (end 177 155.12) (width 0.2) (layer "F.Cu") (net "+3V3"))
 (via (at 167.9 146.5) (size 0.6) (drill 0.3) (layers "F.Cu" "B.Cu") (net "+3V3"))
 (via (at 167.075735 130.075735) (size 0.6) (drill 0.3) (layers "F.Cu" "B.Cu") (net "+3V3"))
 (via (at 167.9 128) (size 0.6) (drill 0.3) (layers "F.Cu" "B.Cu") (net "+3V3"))
 (segment (start 159.5 99.81) (end 167.23 107.54) (width 0.2) (layer "B.Cu") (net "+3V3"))
 (segment (start 167.23 127.33) (end 167.9 128) (width 0.2) (layer "B.Cu") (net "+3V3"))
 (segment (start 159.5 83.5) (end 159.5 99.81) (width 0.2) (layer "B.Cu") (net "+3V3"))
 (segment (start 167.9 130.9) (end 167.9 146.5) (width 0.2) (layer "B.Cu") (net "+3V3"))
 (segment (start 167.23 107.54) (end 167.23 127.33) (width 0.2) (layer "B.Cu") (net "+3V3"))
 (segment (start 167.075735 130.075735) (end 167.9 130.9) (width 0.2) (layer "B.Cu") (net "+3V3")))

